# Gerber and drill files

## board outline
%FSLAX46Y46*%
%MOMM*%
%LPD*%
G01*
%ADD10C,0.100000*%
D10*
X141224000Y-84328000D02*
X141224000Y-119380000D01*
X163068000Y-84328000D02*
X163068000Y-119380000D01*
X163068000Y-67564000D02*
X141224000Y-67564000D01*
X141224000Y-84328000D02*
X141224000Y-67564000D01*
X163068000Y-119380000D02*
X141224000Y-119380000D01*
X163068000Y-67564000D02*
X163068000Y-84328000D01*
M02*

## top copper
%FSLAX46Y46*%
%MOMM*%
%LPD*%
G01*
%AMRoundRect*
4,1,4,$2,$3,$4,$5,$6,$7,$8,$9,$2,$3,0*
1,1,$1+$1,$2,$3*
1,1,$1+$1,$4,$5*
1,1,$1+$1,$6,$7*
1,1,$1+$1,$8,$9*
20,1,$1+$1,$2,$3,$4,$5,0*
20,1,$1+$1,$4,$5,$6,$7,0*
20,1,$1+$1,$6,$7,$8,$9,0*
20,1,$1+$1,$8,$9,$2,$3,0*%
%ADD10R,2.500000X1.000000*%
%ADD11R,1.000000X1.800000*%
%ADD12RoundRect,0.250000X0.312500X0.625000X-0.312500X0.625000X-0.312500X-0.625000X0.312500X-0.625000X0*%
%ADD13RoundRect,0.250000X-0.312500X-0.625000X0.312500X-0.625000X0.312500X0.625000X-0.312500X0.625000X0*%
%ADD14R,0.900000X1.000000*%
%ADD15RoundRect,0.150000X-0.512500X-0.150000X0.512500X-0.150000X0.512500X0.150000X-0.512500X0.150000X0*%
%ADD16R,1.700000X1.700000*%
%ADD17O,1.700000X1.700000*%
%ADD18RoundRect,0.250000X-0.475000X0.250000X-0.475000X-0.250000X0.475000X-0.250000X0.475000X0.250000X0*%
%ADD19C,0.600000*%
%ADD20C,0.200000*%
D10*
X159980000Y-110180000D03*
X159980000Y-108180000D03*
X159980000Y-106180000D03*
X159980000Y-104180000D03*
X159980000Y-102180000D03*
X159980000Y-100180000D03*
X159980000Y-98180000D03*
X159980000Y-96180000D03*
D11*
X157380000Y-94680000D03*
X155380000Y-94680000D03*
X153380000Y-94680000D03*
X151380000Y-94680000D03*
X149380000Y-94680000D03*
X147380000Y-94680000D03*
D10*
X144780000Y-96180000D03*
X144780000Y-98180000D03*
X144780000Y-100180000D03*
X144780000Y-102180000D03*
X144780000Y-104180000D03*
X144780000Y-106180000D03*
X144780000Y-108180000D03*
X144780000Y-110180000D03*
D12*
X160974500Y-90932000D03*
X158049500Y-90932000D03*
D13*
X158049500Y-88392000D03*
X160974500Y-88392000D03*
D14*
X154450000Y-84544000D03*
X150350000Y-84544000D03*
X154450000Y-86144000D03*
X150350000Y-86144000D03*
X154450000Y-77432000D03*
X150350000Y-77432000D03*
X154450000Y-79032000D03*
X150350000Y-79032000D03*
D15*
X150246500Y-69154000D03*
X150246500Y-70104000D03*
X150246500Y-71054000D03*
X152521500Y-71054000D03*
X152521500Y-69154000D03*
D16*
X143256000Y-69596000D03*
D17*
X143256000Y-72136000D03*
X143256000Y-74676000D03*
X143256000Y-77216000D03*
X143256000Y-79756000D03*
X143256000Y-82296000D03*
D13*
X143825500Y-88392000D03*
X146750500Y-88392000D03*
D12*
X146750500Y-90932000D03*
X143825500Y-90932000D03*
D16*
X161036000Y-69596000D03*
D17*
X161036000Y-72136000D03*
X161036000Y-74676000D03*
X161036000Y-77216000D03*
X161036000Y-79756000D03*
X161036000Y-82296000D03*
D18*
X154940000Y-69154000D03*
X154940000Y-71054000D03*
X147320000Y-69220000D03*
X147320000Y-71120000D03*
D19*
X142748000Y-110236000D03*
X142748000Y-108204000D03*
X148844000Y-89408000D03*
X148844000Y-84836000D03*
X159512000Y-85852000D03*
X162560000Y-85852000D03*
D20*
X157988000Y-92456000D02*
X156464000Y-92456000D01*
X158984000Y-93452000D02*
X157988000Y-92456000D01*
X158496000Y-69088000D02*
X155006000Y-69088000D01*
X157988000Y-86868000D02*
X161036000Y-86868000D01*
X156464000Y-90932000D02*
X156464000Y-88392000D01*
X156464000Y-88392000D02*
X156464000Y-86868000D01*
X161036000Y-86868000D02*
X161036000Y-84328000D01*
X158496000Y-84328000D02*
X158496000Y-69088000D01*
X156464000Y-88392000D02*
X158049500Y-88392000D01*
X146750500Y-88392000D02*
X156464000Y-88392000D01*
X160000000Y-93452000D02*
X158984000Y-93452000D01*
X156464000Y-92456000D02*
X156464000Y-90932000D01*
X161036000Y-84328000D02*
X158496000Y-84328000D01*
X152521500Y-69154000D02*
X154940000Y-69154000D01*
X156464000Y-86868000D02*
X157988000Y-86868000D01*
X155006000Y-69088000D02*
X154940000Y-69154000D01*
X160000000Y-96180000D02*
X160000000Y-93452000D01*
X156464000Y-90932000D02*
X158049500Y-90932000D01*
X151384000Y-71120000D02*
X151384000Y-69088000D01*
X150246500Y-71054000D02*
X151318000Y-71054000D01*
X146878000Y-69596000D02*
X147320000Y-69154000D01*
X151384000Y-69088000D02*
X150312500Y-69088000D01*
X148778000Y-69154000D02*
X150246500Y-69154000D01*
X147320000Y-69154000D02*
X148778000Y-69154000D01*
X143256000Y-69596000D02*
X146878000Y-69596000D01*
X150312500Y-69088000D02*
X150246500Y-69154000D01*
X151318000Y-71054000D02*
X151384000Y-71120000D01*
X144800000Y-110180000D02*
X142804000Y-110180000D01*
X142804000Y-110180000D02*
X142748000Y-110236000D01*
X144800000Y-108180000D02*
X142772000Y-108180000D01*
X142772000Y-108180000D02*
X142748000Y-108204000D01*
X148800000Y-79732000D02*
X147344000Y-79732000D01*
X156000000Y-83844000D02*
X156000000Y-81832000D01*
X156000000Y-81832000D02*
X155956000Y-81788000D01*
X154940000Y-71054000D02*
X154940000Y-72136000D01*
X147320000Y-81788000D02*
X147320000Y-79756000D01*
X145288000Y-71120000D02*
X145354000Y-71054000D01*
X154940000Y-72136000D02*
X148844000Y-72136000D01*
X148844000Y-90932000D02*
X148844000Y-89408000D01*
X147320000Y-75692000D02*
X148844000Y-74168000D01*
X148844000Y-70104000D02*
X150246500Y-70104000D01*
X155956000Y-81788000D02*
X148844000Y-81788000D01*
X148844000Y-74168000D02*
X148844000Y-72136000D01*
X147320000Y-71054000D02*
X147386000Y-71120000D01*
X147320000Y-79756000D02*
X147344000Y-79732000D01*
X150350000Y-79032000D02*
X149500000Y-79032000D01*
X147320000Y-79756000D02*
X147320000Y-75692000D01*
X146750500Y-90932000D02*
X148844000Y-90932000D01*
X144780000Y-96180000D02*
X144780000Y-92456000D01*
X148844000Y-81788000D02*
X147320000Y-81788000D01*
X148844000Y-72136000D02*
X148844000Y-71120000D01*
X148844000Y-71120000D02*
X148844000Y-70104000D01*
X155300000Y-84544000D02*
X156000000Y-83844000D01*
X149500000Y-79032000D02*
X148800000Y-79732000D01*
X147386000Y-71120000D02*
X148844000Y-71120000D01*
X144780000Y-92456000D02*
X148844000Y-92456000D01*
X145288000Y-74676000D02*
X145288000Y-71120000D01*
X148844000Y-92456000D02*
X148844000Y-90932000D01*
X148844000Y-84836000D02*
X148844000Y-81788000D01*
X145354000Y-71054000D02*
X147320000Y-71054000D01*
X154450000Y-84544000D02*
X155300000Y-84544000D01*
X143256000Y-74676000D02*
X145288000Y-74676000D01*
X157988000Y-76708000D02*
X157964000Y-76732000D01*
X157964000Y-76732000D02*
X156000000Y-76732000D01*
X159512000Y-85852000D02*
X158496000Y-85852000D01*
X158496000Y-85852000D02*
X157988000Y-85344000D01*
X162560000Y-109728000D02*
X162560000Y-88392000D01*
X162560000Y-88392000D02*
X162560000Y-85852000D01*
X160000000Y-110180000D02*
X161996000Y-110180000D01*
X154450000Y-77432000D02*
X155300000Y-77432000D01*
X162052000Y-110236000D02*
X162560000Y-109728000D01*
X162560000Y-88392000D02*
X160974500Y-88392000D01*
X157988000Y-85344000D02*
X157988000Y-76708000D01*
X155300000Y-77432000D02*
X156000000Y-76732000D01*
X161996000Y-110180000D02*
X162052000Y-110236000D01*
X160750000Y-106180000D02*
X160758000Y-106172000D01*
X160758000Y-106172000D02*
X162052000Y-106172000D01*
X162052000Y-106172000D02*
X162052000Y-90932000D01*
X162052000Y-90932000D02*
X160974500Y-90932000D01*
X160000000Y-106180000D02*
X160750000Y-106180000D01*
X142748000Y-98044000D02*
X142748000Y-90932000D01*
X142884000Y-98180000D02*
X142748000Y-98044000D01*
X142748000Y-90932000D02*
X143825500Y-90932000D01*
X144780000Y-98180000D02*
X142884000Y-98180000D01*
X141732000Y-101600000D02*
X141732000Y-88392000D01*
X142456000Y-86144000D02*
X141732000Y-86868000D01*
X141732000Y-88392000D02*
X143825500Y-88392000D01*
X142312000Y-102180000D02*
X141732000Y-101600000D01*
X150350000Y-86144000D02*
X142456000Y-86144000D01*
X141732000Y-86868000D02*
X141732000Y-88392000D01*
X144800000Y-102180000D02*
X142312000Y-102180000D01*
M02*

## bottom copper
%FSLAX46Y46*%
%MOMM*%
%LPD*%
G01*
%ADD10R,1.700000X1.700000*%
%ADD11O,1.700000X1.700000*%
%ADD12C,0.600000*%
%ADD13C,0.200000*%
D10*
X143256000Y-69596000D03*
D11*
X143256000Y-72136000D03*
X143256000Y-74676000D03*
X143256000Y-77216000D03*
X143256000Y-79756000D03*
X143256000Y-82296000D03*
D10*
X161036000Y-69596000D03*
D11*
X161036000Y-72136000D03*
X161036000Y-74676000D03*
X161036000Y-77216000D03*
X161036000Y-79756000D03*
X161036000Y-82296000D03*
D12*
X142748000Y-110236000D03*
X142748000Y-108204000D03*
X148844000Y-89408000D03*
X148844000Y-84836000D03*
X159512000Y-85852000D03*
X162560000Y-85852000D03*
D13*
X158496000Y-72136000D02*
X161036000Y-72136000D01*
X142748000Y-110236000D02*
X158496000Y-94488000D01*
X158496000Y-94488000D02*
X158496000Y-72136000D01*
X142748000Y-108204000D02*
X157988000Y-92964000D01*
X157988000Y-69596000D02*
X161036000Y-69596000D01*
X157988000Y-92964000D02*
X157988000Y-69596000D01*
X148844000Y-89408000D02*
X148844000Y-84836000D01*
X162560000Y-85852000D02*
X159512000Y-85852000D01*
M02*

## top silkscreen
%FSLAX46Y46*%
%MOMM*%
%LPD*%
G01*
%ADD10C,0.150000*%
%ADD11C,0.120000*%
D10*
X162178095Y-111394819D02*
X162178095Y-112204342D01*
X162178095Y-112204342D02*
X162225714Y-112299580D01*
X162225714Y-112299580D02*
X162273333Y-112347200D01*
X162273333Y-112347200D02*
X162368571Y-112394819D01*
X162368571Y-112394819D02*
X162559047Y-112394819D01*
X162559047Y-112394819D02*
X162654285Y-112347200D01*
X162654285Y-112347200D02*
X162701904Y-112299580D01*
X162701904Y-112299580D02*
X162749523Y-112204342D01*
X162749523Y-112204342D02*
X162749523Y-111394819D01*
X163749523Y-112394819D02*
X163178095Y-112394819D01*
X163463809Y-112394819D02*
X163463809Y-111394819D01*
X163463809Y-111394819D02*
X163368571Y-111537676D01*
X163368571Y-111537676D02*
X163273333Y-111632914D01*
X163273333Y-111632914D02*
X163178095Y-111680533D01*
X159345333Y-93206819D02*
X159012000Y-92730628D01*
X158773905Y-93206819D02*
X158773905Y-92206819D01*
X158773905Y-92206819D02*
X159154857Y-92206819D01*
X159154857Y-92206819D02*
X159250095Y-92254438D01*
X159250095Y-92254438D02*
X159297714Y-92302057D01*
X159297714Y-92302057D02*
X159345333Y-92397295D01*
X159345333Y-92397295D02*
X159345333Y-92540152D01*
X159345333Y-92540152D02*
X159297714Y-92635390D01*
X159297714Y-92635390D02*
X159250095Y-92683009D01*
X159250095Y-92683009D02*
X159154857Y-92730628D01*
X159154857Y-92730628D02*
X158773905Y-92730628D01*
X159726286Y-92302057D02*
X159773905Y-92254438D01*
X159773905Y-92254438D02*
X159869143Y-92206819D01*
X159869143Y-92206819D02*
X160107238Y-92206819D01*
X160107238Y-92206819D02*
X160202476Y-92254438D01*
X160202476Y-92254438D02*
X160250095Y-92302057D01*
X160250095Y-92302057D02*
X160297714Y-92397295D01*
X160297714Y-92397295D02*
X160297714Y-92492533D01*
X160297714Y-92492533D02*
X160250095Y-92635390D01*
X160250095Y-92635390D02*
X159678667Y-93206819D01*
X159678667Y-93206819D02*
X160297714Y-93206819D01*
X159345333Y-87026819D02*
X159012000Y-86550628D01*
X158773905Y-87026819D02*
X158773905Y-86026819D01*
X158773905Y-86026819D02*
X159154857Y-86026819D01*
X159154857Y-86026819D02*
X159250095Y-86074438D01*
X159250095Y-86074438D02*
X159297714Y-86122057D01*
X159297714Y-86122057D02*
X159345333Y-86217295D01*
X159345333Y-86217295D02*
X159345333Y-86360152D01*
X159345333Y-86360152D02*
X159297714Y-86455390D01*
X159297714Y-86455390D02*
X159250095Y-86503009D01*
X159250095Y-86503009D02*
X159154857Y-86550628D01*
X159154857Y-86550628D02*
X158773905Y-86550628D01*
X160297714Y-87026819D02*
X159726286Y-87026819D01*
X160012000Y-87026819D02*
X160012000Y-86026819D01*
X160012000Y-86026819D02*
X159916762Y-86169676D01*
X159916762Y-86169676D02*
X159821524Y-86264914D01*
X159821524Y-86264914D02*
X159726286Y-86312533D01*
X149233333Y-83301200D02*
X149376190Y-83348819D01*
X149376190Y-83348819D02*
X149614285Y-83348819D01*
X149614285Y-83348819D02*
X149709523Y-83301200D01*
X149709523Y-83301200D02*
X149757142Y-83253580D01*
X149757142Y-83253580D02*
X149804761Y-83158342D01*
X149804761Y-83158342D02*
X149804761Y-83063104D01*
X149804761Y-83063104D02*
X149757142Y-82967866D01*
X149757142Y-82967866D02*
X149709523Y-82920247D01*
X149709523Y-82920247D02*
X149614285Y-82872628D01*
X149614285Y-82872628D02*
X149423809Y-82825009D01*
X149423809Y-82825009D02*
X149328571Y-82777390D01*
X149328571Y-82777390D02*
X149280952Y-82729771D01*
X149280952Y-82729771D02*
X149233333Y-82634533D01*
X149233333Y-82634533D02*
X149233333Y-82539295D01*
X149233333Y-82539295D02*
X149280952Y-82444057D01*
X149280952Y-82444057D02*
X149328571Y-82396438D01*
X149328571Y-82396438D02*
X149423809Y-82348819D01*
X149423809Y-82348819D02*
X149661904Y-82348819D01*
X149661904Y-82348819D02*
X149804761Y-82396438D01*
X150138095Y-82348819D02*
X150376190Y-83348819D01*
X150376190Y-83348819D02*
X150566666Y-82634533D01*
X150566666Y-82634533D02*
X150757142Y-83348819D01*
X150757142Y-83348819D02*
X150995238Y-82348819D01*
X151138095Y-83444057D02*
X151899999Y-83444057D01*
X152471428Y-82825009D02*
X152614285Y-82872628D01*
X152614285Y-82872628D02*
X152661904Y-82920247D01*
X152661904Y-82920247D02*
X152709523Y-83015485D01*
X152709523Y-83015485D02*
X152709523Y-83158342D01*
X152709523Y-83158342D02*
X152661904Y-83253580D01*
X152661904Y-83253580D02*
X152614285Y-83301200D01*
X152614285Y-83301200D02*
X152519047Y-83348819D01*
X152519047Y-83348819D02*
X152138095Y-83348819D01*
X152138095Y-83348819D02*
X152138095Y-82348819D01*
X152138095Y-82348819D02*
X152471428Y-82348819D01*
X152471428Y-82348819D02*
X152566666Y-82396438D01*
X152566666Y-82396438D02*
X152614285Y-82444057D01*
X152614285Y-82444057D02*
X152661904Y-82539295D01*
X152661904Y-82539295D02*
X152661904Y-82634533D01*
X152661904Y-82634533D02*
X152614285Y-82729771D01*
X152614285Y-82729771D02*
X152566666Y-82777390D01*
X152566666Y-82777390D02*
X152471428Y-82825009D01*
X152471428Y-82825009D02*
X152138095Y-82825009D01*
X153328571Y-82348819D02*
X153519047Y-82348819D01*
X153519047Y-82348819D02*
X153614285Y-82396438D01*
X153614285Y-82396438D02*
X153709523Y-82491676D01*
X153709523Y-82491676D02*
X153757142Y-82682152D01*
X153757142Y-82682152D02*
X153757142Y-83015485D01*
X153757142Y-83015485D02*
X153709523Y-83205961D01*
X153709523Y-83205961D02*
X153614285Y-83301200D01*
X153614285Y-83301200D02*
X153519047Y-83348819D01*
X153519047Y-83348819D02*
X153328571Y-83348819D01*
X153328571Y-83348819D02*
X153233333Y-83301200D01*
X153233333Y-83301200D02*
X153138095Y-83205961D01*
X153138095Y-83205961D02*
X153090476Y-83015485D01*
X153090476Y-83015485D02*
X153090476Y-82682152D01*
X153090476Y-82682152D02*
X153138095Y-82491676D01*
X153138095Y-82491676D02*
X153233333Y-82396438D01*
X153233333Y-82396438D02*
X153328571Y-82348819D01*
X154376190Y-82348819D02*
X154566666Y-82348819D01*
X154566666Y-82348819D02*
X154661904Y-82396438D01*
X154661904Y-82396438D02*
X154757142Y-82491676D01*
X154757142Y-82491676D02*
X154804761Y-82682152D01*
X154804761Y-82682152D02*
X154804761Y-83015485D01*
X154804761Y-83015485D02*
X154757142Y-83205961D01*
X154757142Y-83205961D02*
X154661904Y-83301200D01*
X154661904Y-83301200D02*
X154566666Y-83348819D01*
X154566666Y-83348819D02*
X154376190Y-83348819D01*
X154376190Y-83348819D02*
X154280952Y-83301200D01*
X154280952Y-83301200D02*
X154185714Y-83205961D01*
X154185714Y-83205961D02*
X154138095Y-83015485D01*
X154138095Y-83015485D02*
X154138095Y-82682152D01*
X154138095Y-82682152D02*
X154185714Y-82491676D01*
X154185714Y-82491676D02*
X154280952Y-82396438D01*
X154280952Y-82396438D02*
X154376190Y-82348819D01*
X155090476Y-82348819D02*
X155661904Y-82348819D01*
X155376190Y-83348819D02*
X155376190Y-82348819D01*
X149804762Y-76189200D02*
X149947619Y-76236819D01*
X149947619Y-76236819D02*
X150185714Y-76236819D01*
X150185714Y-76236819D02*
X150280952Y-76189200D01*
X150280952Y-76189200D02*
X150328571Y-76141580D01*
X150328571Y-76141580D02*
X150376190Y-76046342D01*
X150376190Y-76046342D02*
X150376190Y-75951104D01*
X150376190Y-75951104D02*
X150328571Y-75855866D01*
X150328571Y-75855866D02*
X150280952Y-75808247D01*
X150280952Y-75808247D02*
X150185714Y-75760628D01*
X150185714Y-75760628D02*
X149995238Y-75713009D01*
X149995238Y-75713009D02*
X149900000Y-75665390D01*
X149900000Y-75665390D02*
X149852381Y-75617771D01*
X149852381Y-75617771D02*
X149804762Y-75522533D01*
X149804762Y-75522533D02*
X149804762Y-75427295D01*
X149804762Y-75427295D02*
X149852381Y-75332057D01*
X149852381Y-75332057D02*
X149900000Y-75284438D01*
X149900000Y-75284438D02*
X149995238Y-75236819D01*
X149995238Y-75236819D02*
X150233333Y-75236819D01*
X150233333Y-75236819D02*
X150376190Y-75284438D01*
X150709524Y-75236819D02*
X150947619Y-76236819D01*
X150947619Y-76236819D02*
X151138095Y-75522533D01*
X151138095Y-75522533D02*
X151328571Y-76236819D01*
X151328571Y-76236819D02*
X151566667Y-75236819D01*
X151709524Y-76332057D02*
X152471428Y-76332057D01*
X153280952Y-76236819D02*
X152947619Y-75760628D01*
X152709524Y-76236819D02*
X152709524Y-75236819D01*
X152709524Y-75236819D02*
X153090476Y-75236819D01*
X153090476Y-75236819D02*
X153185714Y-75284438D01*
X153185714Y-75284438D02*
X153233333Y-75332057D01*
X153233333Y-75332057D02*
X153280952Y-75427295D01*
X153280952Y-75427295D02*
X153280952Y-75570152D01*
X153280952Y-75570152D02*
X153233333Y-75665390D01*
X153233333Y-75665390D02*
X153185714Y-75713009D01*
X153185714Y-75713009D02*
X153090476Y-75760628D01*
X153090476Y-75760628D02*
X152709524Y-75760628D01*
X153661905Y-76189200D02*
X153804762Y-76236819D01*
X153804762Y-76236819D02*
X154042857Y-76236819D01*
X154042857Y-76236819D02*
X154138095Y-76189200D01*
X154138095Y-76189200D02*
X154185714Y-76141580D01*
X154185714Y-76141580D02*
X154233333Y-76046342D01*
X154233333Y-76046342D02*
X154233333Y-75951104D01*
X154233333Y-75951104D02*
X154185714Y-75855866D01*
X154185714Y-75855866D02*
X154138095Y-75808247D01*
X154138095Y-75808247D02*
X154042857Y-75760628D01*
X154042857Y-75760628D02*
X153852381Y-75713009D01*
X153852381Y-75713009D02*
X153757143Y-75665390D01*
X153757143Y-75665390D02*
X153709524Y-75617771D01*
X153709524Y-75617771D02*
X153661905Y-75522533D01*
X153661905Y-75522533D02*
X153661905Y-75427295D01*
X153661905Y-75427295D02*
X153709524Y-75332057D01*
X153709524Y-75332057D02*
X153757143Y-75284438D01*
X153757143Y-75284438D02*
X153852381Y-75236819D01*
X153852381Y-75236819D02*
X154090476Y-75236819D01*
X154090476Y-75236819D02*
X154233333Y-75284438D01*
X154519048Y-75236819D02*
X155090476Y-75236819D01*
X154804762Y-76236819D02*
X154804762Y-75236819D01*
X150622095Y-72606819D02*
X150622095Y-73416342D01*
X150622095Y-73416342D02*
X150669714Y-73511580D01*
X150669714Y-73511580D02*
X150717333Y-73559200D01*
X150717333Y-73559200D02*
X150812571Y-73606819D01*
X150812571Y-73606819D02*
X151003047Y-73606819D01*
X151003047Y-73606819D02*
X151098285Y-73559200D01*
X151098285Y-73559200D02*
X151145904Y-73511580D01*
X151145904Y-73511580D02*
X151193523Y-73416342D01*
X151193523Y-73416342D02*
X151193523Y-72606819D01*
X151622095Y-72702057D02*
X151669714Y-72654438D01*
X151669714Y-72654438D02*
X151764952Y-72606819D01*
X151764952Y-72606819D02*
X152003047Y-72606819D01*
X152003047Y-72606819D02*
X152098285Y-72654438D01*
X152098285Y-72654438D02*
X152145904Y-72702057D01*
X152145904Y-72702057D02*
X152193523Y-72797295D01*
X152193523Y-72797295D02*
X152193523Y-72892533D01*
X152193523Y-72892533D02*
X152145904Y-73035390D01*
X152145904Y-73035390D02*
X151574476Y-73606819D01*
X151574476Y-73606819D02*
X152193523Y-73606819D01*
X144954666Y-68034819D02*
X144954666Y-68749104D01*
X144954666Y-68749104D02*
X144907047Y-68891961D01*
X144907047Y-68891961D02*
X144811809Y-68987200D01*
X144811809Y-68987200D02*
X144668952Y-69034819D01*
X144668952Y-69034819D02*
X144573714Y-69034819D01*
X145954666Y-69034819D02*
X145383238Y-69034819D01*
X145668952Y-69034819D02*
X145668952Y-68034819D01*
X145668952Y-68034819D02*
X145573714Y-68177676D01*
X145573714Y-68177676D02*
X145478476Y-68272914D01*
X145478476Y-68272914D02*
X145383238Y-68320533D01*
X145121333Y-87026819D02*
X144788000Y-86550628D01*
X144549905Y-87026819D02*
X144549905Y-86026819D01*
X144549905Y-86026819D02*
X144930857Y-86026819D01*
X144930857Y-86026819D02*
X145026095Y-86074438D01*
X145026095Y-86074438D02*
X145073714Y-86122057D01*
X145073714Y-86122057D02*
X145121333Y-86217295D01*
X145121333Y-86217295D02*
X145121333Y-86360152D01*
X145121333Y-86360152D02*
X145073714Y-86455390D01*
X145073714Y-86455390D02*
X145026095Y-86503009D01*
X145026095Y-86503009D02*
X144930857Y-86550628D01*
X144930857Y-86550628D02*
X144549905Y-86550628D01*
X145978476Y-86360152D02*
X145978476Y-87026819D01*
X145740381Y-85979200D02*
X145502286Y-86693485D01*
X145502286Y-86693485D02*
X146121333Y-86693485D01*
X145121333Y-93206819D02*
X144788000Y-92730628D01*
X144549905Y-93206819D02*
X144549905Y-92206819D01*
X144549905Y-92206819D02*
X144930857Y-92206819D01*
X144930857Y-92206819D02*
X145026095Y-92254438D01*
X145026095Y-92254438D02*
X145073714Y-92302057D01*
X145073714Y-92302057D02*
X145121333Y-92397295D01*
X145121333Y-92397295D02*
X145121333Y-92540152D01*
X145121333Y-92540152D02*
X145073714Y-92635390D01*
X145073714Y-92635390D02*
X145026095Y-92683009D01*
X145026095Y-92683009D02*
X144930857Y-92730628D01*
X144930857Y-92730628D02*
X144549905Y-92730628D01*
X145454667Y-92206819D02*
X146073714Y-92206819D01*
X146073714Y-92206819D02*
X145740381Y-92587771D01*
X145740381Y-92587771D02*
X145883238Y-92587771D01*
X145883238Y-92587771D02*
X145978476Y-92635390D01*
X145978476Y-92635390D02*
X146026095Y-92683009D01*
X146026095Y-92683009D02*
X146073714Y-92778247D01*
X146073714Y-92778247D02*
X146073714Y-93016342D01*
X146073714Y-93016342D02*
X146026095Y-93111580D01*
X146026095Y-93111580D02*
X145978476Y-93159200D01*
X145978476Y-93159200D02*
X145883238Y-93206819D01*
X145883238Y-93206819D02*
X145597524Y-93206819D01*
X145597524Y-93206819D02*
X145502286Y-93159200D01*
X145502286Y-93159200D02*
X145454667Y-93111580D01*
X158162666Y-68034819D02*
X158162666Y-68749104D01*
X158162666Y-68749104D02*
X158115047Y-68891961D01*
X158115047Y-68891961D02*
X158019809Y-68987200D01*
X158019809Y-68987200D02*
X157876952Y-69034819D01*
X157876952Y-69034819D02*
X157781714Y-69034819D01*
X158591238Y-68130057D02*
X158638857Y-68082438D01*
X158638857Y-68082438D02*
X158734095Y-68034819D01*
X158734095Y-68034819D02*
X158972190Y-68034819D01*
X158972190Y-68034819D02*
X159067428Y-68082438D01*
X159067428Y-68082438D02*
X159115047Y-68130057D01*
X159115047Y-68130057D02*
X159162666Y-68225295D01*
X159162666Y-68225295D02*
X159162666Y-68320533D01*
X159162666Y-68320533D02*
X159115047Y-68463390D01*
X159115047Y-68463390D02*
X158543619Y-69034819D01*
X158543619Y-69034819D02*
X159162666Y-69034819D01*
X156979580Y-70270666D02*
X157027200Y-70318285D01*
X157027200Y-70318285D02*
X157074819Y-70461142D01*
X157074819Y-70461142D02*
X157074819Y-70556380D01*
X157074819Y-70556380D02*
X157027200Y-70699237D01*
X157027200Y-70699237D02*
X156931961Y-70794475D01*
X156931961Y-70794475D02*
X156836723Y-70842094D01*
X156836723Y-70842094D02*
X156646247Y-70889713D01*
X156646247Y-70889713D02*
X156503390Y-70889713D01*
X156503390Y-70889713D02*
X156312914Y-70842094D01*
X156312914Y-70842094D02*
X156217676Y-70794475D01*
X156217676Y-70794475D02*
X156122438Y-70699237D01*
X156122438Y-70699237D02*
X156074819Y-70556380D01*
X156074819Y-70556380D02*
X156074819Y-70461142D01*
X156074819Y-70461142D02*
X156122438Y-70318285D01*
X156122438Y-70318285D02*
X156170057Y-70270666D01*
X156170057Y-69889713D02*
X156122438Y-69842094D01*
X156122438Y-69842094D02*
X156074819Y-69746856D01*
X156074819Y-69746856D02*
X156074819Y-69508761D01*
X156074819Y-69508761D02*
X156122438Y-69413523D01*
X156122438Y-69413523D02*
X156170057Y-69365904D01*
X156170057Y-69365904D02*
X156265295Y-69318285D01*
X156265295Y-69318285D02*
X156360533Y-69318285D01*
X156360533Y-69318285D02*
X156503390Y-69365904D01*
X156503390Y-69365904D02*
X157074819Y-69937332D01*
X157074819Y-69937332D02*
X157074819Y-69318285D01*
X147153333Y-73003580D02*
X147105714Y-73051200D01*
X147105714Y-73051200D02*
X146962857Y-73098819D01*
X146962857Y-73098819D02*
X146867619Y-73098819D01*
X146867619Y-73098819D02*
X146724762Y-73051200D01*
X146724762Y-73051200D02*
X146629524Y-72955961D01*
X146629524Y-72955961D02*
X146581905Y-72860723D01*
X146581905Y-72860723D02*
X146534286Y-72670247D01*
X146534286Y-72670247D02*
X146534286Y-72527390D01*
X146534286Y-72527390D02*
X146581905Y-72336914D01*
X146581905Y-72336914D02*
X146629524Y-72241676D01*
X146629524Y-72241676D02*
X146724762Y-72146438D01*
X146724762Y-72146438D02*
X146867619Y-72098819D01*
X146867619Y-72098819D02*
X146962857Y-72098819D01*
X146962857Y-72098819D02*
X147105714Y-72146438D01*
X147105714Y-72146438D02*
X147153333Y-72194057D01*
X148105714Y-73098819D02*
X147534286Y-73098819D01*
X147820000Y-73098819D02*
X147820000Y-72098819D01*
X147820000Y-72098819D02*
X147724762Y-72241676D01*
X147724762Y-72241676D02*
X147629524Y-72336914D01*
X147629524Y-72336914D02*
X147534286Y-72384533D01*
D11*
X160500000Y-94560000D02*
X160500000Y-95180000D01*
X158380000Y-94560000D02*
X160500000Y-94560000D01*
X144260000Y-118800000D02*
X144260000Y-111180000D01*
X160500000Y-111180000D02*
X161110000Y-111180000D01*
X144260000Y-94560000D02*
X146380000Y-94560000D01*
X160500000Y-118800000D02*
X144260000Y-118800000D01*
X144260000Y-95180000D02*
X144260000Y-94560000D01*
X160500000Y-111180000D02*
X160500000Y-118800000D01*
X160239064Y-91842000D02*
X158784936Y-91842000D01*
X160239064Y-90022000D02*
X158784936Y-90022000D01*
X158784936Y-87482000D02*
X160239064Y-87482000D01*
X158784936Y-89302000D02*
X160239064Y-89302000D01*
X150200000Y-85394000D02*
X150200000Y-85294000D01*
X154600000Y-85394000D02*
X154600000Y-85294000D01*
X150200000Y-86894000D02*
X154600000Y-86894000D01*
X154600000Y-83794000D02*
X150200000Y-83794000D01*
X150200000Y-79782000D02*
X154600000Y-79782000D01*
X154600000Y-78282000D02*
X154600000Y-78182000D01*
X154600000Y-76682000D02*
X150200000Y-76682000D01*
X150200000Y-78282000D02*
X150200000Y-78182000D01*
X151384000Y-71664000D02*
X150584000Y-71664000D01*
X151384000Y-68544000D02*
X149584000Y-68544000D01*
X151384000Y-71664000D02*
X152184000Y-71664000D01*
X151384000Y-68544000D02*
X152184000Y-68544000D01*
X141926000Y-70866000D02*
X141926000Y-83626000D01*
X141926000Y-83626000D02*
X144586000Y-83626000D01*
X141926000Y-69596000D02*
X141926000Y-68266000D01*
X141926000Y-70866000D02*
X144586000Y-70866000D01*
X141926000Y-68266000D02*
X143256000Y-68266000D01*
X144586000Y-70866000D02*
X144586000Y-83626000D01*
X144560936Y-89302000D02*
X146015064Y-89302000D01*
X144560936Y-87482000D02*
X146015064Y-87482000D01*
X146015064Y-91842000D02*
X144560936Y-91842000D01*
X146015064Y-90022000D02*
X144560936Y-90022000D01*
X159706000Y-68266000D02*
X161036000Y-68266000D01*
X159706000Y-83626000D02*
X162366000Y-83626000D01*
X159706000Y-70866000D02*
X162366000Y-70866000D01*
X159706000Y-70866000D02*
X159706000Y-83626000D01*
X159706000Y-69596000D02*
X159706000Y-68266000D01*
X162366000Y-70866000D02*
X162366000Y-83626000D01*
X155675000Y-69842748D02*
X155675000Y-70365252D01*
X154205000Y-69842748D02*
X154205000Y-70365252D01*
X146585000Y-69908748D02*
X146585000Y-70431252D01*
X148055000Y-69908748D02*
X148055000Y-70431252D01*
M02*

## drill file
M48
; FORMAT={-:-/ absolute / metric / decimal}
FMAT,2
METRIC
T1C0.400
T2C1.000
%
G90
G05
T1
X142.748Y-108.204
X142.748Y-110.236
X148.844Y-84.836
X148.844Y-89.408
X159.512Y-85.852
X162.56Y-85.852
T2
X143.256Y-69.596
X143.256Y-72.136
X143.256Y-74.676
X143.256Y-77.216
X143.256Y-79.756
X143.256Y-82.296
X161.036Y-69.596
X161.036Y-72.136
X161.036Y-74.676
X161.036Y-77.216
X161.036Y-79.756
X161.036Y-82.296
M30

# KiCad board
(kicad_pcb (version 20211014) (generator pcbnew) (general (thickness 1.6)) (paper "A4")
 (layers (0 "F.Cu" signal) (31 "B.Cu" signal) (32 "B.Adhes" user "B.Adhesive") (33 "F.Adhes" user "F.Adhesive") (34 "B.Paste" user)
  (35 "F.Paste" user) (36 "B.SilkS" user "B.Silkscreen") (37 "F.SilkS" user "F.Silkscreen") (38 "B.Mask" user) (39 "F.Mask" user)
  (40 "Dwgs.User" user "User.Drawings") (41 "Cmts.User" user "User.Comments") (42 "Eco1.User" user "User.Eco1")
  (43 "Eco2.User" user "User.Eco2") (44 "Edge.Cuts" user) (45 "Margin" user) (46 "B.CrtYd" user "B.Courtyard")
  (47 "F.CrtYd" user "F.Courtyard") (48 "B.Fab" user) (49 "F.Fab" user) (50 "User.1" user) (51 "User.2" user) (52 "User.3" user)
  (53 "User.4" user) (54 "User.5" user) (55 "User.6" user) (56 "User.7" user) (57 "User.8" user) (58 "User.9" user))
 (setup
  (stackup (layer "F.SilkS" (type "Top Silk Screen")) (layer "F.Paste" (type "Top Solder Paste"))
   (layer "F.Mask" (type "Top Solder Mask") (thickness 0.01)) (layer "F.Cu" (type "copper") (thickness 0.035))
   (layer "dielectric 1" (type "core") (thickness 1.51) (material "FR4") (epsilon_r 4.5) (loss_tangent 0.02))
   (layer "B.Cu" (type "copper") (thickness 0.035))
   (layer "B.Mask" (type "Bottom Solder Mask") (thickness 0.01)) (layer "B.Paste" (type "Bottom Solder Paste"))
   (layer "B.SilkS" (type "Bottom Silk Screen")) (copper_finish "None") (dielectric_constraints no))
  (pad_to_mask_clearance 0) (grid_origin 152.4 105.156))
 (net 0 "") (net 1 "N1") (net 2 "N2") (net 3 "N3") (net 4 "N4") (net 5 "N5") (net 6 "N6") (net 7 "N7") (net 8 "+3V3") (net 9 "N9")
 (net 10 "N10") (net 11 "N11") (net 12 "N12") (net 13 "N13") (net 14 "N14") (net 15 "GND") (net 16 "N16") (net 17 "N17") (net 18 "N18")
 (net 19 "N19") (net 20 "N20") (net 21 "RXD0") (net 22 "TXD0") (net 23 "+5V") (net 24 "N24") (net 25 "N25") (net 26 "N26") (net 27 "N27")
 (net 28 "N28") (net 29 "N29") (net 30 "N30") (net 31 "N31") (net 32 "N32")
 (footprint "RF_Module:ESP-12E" (layer "F.Cu") (at 152.38 106.68 180)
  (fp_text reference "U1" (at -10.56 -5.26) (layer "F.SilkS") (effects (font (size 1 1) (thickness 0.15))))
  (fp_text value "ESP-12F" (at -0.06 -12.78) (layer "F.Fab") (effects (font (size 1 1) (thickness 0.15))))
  (fp_line (start -8.12 12.12) (end -8.12 11.5) (layer "F.SilkS") (width 0.12))
  (fp_line (start -6 12.12) (end -8.12 12.12) (layer "F.SilkS") (width 0.12))
  (fp_line (start 8.12 -12.12) (end 8.12 -4.5) (layer "F.SilkS") (width 0.12))
  (fp_line (start -8.12 -4.5) (end -8.73 -4.5) (layer "F.SilkS") (width 0.12))
  (fp_line (start 8.12 12.12) (end 6 12.12) (layer "F.SilkS") (width 0.12))
  (fp_line (start -8.12 -12.12) (end 8.12 -12.12) (layer "F.SilkS") (width 0.12))
  (fp_line (start 8.12 11.5) (end 8.12 12.12) (layer "F.SilkS") (width 0.12))
  (fp_line (start -8.12 -4.5) (end -8.12 -12.12) (layer "F.SilkS") (width 0.12))
  (pad "1" smd rect (at -7.6 -3.5 180) (size 2.5 1) (layers "F.Cu" "F.Paste" "F.Mask") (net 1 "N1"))
  (pad "2" smd rect (at -7.6 -1.5 180) (size 2.5 1) (layers "F.Cu" "F.Paste" "F.Mask") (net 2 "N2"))
  (pad "3" smd rect (at -7.6 0.5 180) (size 2.5 1) (layers "F.Cu" "F.Paste" "F.Mask") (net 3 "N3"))
  (pad "4" smd rect (at -7.6 2.5 180) (size 2.5 1) (layers "F.Cu" "F.Paste" "F.Mask") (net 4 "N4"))
  (pad "5" smd rect (at -7.6 4.5 180) (size 2.5 1) (layers "F.Cu" "F.Paste" "F.Mask") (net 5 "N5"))
  (pad "6" smd rect (at -7.6 6.5 180) (size 2.5 1) (layers "F.Cu" "F.Paste" "F.Mask") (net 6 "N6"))
  (pad "7" smd rect (at -7.6 8.5 180) (size 2.5 1) (layers "F.Cu" "F.Paste" "F.Mask") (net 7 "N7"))
  (pad "8" smd rect (at -7.6 10.5 180) (size 2.5 1) (layers "F.Cu" "F.Paste" "F.Mask") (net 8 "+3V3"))
  (pad "9" smd rect (at -5 12 180) (size 1 1.8) (layers "F.Cu" "F.Paste" "F.Mask") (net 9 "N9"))
  (pad "10" smd rect (at -3 12 180) (size 1 1.8) (layers "F.Cu" "F.Paste" "F.Mask") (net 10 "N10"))
  (pad "11" smd rect (at -1 12 180) (size 1 1.8) (layers "F.Cu" "F.Paste" "F.Mask") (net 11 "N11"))
  (pad "12" smd rect (at 1 12 180) (size 1 1.8) (layers "F.Cu" "F.Paste" "F.Mask") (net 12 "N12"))
  (pad "13" smd rect (at 3 12 180) (size 1 1.8) (layers "F.Cu" "F.Paste" "F.Mask") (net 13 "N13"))
  (pad "14" smd rect (at 5 12 180) (size 1 1.8) (layers "F.Cu" "F.Paste" "F.Mask") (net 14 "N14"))
  (pad "15" smd rect (at 7.6 10.5 180) (size 2.5 1) (layers "F.Cu" "F.Paste" "F.Mask") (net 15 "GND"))
  (pad "16" smd rect (at 7.6 8.5 180) (size 2.5 1) (layers "F.Cu" "F.Paste" "F.Mask") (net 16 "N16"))
  (pad "17" smd rect (at 7.6 6.5 180) (size 2.5 1) (layers "F.Cu" "F.Paste" "F.Mask") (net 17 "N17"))
  (pad "18" smd rect (at 7.6 4.5 180) (size 2.5 1) (layers "F.Cu" "F.Paste" "F.Mask") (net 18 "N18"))
  (pad "19" smd rect (at 7.6 2.5 180) (size 2.5 1) (layers "F.Cu" "F.Paste" "F.Mask") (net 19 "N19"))
  (pad "20" smd rect (at 7.6 0.5 180) (size 2.5 1) (layers "F.Cu" "F.Paste" "F.Mask") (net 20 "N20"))
  (pad "21" smd rect (at 7.6 -1.5 180) (size 2.5 1) (layers "F.Cu" "F.Paste" "F.Mask") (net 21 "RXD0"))
  (pad "22" smd rect (at 7.6 -3.5 180) (size 2.5 1) (layers "F.Cu" "F.Paste" "F.Mask") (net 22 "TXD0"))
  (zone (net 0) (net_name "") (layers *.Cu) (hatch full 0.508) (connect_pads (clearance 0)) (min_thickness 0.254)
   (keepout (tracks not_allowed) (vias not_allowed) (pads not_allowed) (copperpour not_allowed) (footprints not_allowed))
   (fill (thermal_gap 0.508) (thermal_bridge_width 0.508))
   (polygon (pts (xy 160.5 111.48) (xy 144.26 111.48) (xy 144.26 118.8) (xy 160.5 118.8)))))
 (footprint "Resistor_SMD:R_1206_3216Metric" (layer "F.Cu") (at 159.512 90.932 180)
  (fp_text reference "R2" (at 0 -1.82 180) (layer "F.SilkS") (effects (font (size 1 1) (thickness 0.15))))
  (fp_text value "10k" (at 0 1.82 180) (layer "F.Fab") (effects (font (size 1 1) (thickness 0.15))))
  (fp_line (start -0.727064 -0.91) (end 0.727064 -0.91) (layer "F.SilkS") (width 0.12))
  (fp_line (start -0.727064 0.91) (end 0.727064 0.91) (layer "F.SilkS") (width 0.12))
  (pad "1" smd roundrect (at -1.4625 0 180) (size 1.125 1.75) (layers "F.Cu" "F.Paste" "F.Mask") (roundrect_rratio 0.2222222222)
   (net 3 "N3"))
  (pad "2" smd roundrect (at 1.4625 0 180) (size 1.125 1.75) (layers "F.Cu" "F.Paste" "F.Mask") (roundrect_rratio 0.2222222222)
   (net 8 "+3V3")))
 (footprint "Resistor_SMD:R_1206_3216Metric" (layer "F.Cu") (at 159.512 88.392)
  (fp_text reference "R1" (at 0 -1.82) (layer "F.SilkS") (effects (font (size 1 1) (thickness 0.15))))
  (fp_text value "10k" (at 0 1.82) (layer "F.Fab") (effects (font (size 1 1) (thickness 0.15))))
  (fp_line (start -0.727064 -0.91) (end 0.727064 -0.91) (layer "F.SilkS") (width 0.12))
  (fp_line (start -0.727064 0.91) (end 0.727064 0.91) (layer "F.SilkS") (width 0.12))
  (pad "1" smd roundrect (at -1.4625 0) (size 1.125 1.75) (layers "F.Cu" "F.Paste" "F.Mask") (roundrect_rratio 0.2222222222) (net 8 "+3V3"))
  (pad "2" smd roundrect (at 1.4625 0) (size 1.125 1.75) (layers "F.Cu" "F.Paste" "F.Mask") (roundrect_rratio 0.2222222222) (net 1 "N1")))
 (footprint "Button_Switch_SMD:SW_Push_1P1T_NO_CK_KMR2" (layer "F.Cu") (at 152.4 85.344)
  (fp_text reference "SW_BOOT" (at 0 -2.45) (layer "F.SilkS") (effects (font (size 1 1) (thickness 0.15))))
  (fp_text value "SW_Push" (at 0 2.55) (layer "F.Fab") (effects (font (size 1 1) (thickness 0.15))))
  (fp_line (start -2.2 0.05) (end -2.2 -0.05) (layer "F.SilkS") (width 0.12))
  (fp_line (start 2.2 0.05) (end 2.2 -0.05) (layer "F.SilkS") (width 0.12))
  (fp_line (start -2.2 1.55) (end 2.2 1.55) (layer "F.SilkS") (width 0.12))
  (fp_line (start 2.2 -1.55) (end -2.2 -1.55) (layer "F.SilkS") (width 0.12))
  (pad "1" smd rect (at 2.05 -0.8) (size 0.9 1) (layers "F.Cu" "F.Paste" "F.Mask") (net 15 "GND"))
  (pad "1" smd rect (at -2.05 -0.8) (size 0.9 1) (layers "F.Cu" "F.Paste" "F.Mask") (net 15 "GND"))
  (pad "2" smd rect (at 2.05 0.8) (size 0.9 1) (layers "F.Cu" "F.Paste" "F.Mask") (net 18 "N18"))
  (pad "2" smd rect (at -2.05 0.8) (size 0.9 1) (layers "F.Cu" "F.Paste" "F.Mask") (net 18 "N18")))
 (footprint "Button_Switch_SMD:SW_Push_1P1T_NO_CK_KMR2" (layer "F.Cu") (at 152.4 78.232)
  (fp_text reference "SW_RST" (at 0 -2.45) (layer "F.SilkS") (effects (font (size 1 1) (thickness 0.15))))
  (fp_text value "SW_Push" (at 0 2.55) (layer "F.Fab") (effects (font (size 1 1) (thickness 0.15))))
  (fp_line (start -2.2 1.55) (end 2.2 1.55) (layer "F.SilkS") (width 0.12))
  (fp_line (start 2.2 0.05) (end 2.2 -0.05) (layer "F.SilkS") (width 0.12))
  (fp_line (start 2.2 -1.55) (end -2.2 -1.55) (layer "F.SilkS") (width 0.12))
  (fp_line (start -2.2 0.05) (end -2.2 -0.05) (layer "F.SilkS") (width 0.12))
  (pad "1" smd rect (at 2.05 -0.8) (size 0.9 1) (layers "F.Cu" "F.Paste" "F.Mask") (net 1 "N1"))
  (pad "1" smd rect (at -2.05 -0.8) (size 0.9 1) (layers "F.Cu" "F.Paste" "F.Mask") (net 1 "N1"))
  (pad "2" smd rect (at 2.05 0.8) (size 0.9 1) (layers "F.Cu" "F.Paste" "F.Mask") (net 15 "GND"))
  (pad "2" smd rect (at -2.05 0.8) (size 0.9 1) (layers "F.Cu" "F.Paste" "F.Mask") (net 15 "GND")))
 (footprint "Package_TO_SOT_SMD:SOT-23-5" (layer "F.Cu") (at 151.384 70.104)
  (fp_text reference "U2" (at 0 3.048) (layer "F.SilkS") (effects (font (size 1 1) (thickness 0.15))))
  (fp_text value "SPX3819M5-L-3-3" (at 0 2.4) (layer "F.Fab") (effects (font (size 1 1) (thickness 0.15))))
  (fp_line (start 0 1.56) (end -0.8 1.56) (layer "F.SilkS") (width 0.12))
  (fp_line (start 0 -1.56) (end -1.8 -1.56) (layer "F.SilkS") (width 0.12))
  (fp_line (start 0 1.56) (end 0.8 1.56) (layer "F.SilkS") (width 0.12))
  (fp_line (start 0 -1.56) (end 0.8 -1.56) (layer "F.SilkS") (width 0.12))
  (pad "1" smd roundrect (at -1.1375 -0.95) (size 1.325 0.6) (layers "F.Cu" "F.Paste" "F.Mask") (roundrect_rratio 0.25) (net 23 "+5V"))
  (pad "2" smd roundrect (at -1.1375 0) (size 1.325 0.6) (layers "F.Cu" "F.Paste" "F.Mask") (roundrect_rratio 0.25) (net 15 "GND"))
  (pad "3" smd roundrect (at -1.1375 0.95) (size 1.325 0.6) (layers "F.Cu" "F.Paste" "F.Mask") (roundrect_rratio 0.25) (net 23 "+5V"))
  (pad "4" smd roundrect (at 1.1375 0.95) (size 1.325 0.6) (layers "F.Cu" "F.Paste" "F.Mask") (roundrect_rratio 0.25) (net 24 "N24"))
  (pad "5" smd roundrect (at 1.1375 -0.95) (size 1.325 0.6) (layers "F.Cu" "F.Paste" "F.Mask") (roundrect_rratio 0.25) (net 8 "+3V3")))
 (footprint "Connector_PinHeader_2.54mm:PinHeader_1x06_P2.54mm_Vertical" (layer "F.Cu") (at 143.256 69.596)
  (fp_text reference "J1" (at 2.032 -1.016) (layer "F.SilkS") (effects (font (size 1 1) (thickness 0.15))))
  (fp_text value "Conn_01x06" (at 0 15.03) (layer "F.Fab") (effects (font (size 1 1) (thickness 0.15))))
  (fp_line (start -1.33 1.27) (end -1.33 14.03) (layer "F.SilkS") (width 0.12))
  (fp_line (start -1.33 14.03) (end 1.33 14.03) (layer "F.SilkS") (width 0.12))
  (fp_line (start -1.33 0) (end -1.33 -1.33) (layer "F.SilkS") (width 0.12))
  (fp_line (start -1.33 1.27) (end 1.33 1.27) (layer "F.SilkS") (width 0.12))
  (fp_line (start -1.33 -1.33) (end 0 -1.33) (layer "F.SilkS") (width 0.12))
  (fp_line (start 1.33 1.27) (end 1.33 14.03) (layer "F.SilkS") (width 0.12))
  (pad "1" thru_hole rect (at 0 0) (size 1.7 1.7) (drill 1) (layers *.Cu *.Mask) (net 23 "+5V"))
  (pad "2" thru_hole oval (at 0 2.54) (size 1.7 1.7) (drill 1) (layers *.Cu *.Mask) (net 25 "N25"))
  (pad "3" thru_hole oval (at 0 5.08) (size 1.7 1.7) (drill 1) (layers *.Cu *.Mask) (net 15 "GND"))
  (pad "4" thru_hole oval (at 0 7.62) (size 1.7 1.7) (drill 1) (layers *.Cu *.Mask) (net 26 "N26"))
  (pad "5" thru_hole oval (at 0 10.16) (size 1.7 1.7) (drill 1) (layers *.Cu *.Mask) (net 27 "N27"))
  (pad "6" thru_hole oval (at 0 12.7) (size 1.7 1.7) (drill 1) (layers *.Cu *.Mask) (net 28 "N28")))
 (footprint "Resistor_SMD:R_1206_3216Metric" (layer "F.Cu") (at 145.288 88.392)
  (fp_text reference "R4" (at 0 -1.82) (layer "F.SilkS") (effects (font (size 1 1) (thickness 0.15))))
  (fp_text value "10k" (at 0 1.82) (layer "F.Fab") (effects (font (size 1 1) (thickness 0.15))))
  (fp_line (start -0.727064 0.91) (end 0.727064 0.91) (layer "F.SilkS") (width 0.12))
  (fp_line (start -0.727064 -0.91) (end 0.727064 -0.91) (layer "F.SilkS") (width 0.12))
  (pad "1" smd roundrect (at -1.4625 0) (size 1.125 1.75) (layers "F.Cu" "F.Paste" "F.Mask") (roundrect_rratio 0.2222222222) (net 18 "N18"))
  (pad "2" smd roundrect (at 1.4625 0) (size 1.125 1.75) (layers "F.Cu" "F.Paste" "F.Mask") (roundrect_rratio 0.2222222222) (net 8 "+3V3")))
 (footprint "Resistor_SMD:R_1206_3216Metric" (layer "F.Cu") (at 145.288 90.932 180)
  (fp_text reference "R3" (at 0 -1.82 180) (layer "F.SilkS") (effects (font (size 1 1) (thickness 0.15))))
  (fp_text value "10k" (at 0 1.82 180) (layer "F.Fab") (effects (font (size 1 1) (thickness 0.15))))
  (fp_line (start -0.727064 -0.91) (end 0.727064 -0.91) (layer "F.SilkS") (width 0.12))
  (fp_line (start -0.727064 0.91) (end 0.727064 0.91) (layer "F.SilkS") (width 0.12))
  (pad "1" smd roundrect (at -1.4625 0 180) (size 1.125 1.75) (layers "F.Cu" "F.Paste" "F.Mask") (roundrect_rratio 0.2222222222)
   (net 15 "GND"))
  (pad "2" smd roundrect (at 1.4625 0 180) (size 1.125 1.75) (layers "F.Cu" "F.Paste" "F.Mask") (roundrect_rratio 0.2222222222)
   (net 16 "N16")))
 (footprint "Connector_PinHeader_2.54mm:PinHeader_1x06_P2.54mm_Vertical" (layer "F.Cu") (at 161.036 69.596)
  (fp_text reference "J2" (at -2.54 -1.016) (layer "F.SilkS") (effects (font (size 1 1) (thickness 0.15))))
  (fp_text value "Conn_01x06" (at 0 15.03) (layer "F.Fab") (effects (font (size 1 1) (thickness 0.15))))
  (fp_line (start -1.33 -1.33) (end 0 -1.33) (layer "F.SilkS") (width 0.12))
  (fp_line (start -1.33 14.03) (end 1.33 14.03) (layer "F.SilkS") (width 0.12))
  (fp_line (start -1.33 1.27) (end 1.33 1.27) (layer "F.SilkS") (width 0.12))
  (fp_line (start -1.33 1.27) (end -1.33 14.03) (layer "F.SilkS") (width 0.12))
  (fp_line (start -1.33 0) (end -1.33 -1.33) (layer "F.SilkS") (width 0.12))
  (fp_line (start 1.33 1.27) (end 1.33 14.03) (layer "F.SilkS") (width 0.12))
  (pad "1" thru_hole rect (at 0 0) (size 1.7 1.7) (drill 1) (layers *.Cu *.Mask) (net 21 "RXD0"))
  (pad "2" thru_hole oval (at 0 2.54) (size 1.7 1.7) (drill 1) (layers *.Cu *.Mask) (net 22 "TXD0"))
  (pad "3" thru_hole oval (at 0 5.08) (size 1.7 1.7) (drill 1) (layers *.Cu *.Mask) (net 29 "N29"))
  (pad "4" thru_hole oval (at 0 7.62) (size 1.7 1.7) (drill 1) (layers *.Cu *.Mask) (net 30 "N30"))
  (pad "5" thru_hole oval (at 0 10.16) (size 1.7 1.7) (drill 1) (layers *.Cu *.Mask) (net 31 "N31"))
  (pad "6" thru_hole oval (at 0 12.7) (size 1.7 1.7) (drill 1) (layers *.Cu *.Mask) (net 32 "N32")))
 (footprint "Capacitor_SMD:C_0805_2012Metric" (layer "F.Cu") (at 154.94 70.104 -90)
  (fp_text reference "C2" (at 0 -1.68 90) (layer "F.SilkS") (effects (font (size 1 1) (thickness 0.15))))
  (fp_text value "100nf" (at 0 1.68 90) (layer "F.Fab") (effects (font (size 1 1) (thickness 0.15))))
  (fp_line (start -0.261252 -0.735) (end 0.261252 -0.735) (layer "F.SilkS") (width 0.12))
  (fp_line (start -0.261252 0.735) (end 0.261252 0.735) (layer "F.SilkS") (width 0.12))
  (pad "1" smd roundrect (at -0.95 0 270) (size 1 1.45) (layers "F.Cu" "F.Paste" "F.Mask") (roundrect_rratio 0.25) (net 8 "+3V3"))
  (pad "2" smd roundrect (at 0.95 0 270) (size 1 1.45) (layers "F.Cu" "F.Paste" "F.Mask") (roundrect_rratio 0.25) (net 15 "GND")))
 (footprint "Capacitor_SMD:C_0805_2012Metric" (layer "F.Cu") (at 147.32 70.17 -90)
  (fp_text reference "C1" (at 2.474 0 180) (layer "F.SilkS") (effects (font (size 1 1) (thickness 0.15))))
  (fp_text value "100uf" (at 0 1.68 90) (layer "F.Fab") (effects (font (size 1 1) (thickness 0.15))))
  (fp_line (start -0.261252 0.735) (end 0.261252 0.735) (layer "F.SilkS") (width 0.12))
  (fp_line (start -0.261252 -0.735) (end 0.261252 -0.735) (layer "F.SilkS") (width 0.12))
  (pad "1" smd roundrect (at -0.95 0 270) (size 1 1.45) (layers "F.Cu" "F.Paste" "F.Mask") (roundrect_rratio 0.25) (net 23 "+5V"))
  (pad "2" smd roundrect (at 0.95 0 270) (size 1 1.45) (layers "F.Cu" "F.Paste" "F.Mask") (roundrect_rratio 0.25) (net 15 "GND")))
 (gr_line (start 141.224 84.328) (end 141.224 119.38) (layer "Edge.Cuts") (width 0.1))
 (gr_line (start 163.068 84.328) (end 163.068 119.38) (layer "Edge.Cuts") (width 0.1))
 (gr_line (start 163.068 67.564) (end 141.224 67.564) (layer "Edge.Cuts") (width 0.1))
 (gr_line (start 141.224 84.328) (end 141.224 67.564) (layer "Edge.Cuts") (width 0.1))
 (gr_line (start 163.068 119.38) (end 141.224 119.38) (layer "Edge.Cuts") (width 0.1))
 (gr_line (start 163.068 67.564) (end 163.068 84.328) (layer "Edge.Cuts") (width 0.1))
 (segment (start 157.988 92.456) (end 156.464 92.456) (width 0.2) (layer "F.Cu") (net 8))
 (segment (start 158.984 93.452) (end 157.988 92.456) (width 0.2) (layer "F.Cu") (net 8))
 (segment (start 158.496 69.088) (end 155.006 69.088) (width 0.2) (layer "F.Cu") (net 8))
 (segment (start 157.988 86.868) (end 161.036 86.868) (width 0.2) (layer "F.Cu") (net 8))
 (segment (start 156.464 90.932) (end 156.464 88.392) (width 0.2) (layer "F.Cu") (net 8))
 (segment (start 156.464 88.392) (end 156.464 86.868) (width 0.2) (layer "F.Cu") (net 8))
 (segment (start 161.036 86.868) (end 161.036 84.328) (width 0.2) (layer "F.Cu") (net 8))
 (segment (start 158.496 84.328) (end 158.496 69.088) (width 0.2) (layer "F.Cu") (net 8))
 (segment (start 156.464 88.392) (end 158.0495 88.392) (width 0.2) (layer "F.Cu") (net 8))
 (segment (start 146.7505 88.392) (end 156.464 88.392) (width 0.2) (layer "F.Cu") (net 8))
 (segment (start 160 93.452) (end 158.984 93.452) (width 0.2) (layer "F.Cu") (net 8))
 (segment (start 156.464 92.456) (end 156.464 90.932) (width 0.2) (layer "F.Cu") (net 8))
 (segment (start 161.036 84.328) (end 158.496 84.328) (width 0.2) (layer "F.Cu") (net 8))
 (segment (start 152.5215 69.154) (end 154.94 69.154) (width 0.2) (layer "F.Cu") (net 8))
 (segment (start 156.464 86.868) (end 157.988 86.868) (width 0.2) (layer "F.Cu") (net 8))
 (segment (start 155.006 69.088) (end 154.94 69.154) (width 0.2) (layer "F.Cu") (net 8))
 (segment (start 160 96.18) (end 160 93.452) (width 0.2) (layer "F.Cu") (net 8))
 (segment (start 156.464 90.932) (end 158.0495 90.932) (width 0.2) (layer "F.Cu") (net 8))
 (segment (start 151.384 71.12) (end 151.384 69.088) (width 0.2) (layer "F.Cu") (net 23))
 (segment (start 150.2465 71.054) (end 151.318 71.054) (width 0.2) (layer "F.Cu") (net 23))
 (segment (start 146.878 69.596) (end 147.32 69.154) (width 0.2) (layer "F.Cu") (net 23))
 (segment (start 151.384 69.088) (end 150.3125 69.088) (width 0.2) (layer "F.Cu") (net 23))
 (segment (start 148.778 69.154) (end 150.2465 69.154) (width 0.2) (layer "F.Cu") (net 23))
 (segment (start 147.32 69.154) (end 148.778 69.154) (width 0.2) (layer "F.Cu") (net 23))
 (segment (start 143.256 69.596) (end 146.878 69.596) (width 0.2) (layer "F.Cu") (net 23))
 (segment (start 150.3125 69.088) (end 150.2465 69.154) (width 0.2) (layer "F.Cu") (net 23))
 (segment (start 151.318 71.054) (end 151.384 71.12) (width 0.2) (layer "F.Cu") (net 23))
 (segment (start 144.8 110.18) (end 142.804 110.18) (width 0.2) (layer "F.Cu") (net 22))
 (segment (start 142.804 110.18) (end 142.748 110.236) (width 0.2) (layer "F.Cu") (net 22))
 (via (at 142.748 110.236) (size 0.6) (drill 0.4) (layers "F.Cu" "B.Cu") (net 22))
 (segment (start 158.496 72.136) (end 161.036 72.136) (width 0.2) (layer "B.Cu") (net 22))
 (segment (start 142.748 110.236) (end 158.496 94.488) (width 0.2) (layer "B.Cu") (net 22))
 (segment (start 158.496 94.488) (end 158.496 72.136) (width 0.2) (layer "B.Cu") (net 22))
 (segment (start 144.8 108.18) (end 142.772 108.18) (width 0.2) (layer "F.Cu") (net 21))
 (segment (start 142.772 108.18) (end 142.748 108.204) (width 0.2) (layer "F.Cu") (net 21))
 (via (at 142.748 108.204) (size 0.6) (drill 0.4) (layers "F.Cu" "B.Cu") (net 21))
 (segment (start 142.748 108.204) (end 157.988 92.964) (width 0.2) (layer "B.Cu") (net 21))
 (segment (start 157.988 69.596) (end 161.036 69.596) (width 0.2) (layer "B.Cu") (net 21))
 (segment (start 157.988 92.964) (end 157.988 69.596) (width 0.2) (layer "B.Cu") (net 21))
 (segment (start 148.8 79.732) (end 147.344 79.732) (width 0.2) (layer "F.Cu") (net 15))
 (segment (start 156 83.844) (end 156 81.832) (width 0.2) (layer "F.Cu") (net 15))
 (segment (start 156 81.832) (end 155.956 81.788) (width 0.2) (layer "F.Cu") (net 15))
 (segment (start 154.94 71.054) (end 154.94 72.136) (width 0.2) (layer "F.Cu") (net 15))
 (segment (start 147.32 81.788) (end 147.32 79.756) (width 0.2) (layer "F.Cu") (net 15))
 (segment (start 145.288 71.12) (end 145.354 71.054) (width 0.2) (layer "F.Cu") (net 15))
 (segment (start 154.94 72.136) (end 148.844 72.136) (width 0.2) (layer "F.Cu") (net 15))
 (segment (start 148.844 90.932) (end 148.844 89.408) (width 0.2) (layer "F.Cu") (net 15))
 (segment (start 147.32 75.692) (end 148.844 74.168) (width 0.2) (layer "F.Cu") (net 15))
 (segment (start 148.844 70.104) (end 150.2465 70.104) (width 0.2) (layer "F.Cu") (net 15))
 (segment (start 155.956 81.788) (end 148.844 81.788) (width 0.2) (layer "F.Cu") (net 15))
 (segment (start 148.844 74.168) (end 148.844 72.136) (width 0.2) (layer "F.Cu") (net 15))
 (segment (start 147.32 71.054) (end 147.386 71.12) (width 0.2) (layer "F.Cu") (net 15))
 (segment (start 147.32 79.756) (end 147.344 79.732) (width 0.2) (layer "F.Cu") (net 15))
 (segment (start 150.35 79.032) (end 149.5 79.032) (width 0.2) (layer "F.Cu") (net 15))
 (segment (start 147.32 79.756) (end 147.32 75.692) (width 0.2) (layer "F.Cu") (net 15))
 (segment (start 146.7505 90.932) (end 148.844 90.932) (width 0.2) (layer "F.Cu") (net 15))
 (segment (start 144.78 96.18) (end 144.78 92.456) (width 0.2) (layer "F.Cu") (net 15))
 (segment (start 148.844 81.788) (end 147.32 81.788) (width 0.2) (layer "F.Cu") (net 15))
 (segment (start 148.844 72.136) (end 148.844 71.12) (width 0.2) (layer "F.Cu") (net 15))
 (segment (start 148.844 71.12) (end 148.844 70.104) (width 0.2) (layer "F.Cu") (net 15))
 (segment (start 155.3 84.544) (end 156 83.844) (width 0.2) (layer "F.Cu") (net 15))
 (segment (start 149.5 79.032) (end 148.8 79.732) (width 0.2) (layer "F.Cu") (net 15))
 (segment (start 147.386 71.12) (end 148.844 71.12) (width 0.2) (layer "F.Cu") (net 15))
 (segment (start 144.78 92.456) (end 148.844 92.456) (width 0.2) (layer "F.Cu") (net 15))
 (segment (start 145.288 74.676) (end 145.288 71.12) (width 0.2) (layer "F.Cu") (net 15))
 (segment (start 148.844 92.456) (end 148.844 90.932) (width 0.2) (layer "F.Cu") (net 15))
 (segment (start 148.844 84.836) (end 148.844 81.788) (width 0.2) (layer "F.Cu") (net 15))
 (segment (start 145.354 71.054) (end 147.32 71.054) (width 0.2) (layer "F.Cu") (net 15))
 (segment (start 154.45 84.544) (end 155.3 84.544) (width 0.2) (layer "F.Cu") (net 15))
 (segment (start 143.256 74.676) (end 145.288 74.676) (width 0.2) (layer "F.Cu") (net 15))
 (via (at 148.844 89.408) (size 0.6) (drill 0.4) (layers "F.Cu" "B.Cu") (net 15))
 (via (at 148.844 84.836) (size 0.6) (drill 0.4) (layers "F.Cu" "B.Cu") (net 15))
 (segment (start 148.844 89.408) (end 148.844 84.836) (width 0.2) (layer "B.Cu") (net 15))
 (segment (start 157.988 76.708) (end 157.964 76.732) (width 0.2) (layer "F.Cu") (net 1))
 (segment (start 157.964 76.732) (end 156 76.732) (width 0.2) (layer "F.Cu") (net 1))
 (segment (start 159.512 85.852) (end 158.496 85.852) (width 0.2) (layer "F.Cu") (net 1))
 (segment (start 158.496 85.852) (end 157.988 85.344) (width 0.2) (layer "F.Cu") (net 1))
 (segment (start 162.56 109.728) (end 162.56 88.392) (width 0.2) (layer "F.Cu") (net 1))
 (segment (start 162.56 88.392) (end 162.56 85.852) (width 0.2) (layer "F.Cu") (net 1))
 (segment (start 160 110.18) (end 161.996 110.18) (width 0.2) (layer "F.Cu") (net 1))
 (segment (start 154.45 77.432) (end 155.3 77.432) (width 0.2) (layer "F.Cu") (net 1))
 (segment (start 162.052 110.236) (end 162.56 109.728) (width 0.2) (layer "F.Cu") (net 1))
 (segment (start 162.56 88.392) (end 160.9745 88.392) (width 0.2) (layer "F.Cu") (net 1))
 (segment (start 157.988 85.344) (end 157.988 76.708) (width 0.2) (layer "F.Cu") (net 1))
 (segment (start 155.3 77.432) (end 156 76.732) (width 0.2) (layer "F.Cu") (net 1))
 (segment (start 161.996 110.18) (end 162.052 110.236) (width 0.2) (layer "F.Cu") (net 1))
 (via (at 159.512 85.852) (size 0.6) (drill 0.4) (layers "F.Cu" "B.Cu") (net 1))
 (via (at 162.56 85.852) (size 0.6) (drill 0.4) (layers "F.Cu" "B.Cu") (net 1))
 (segment (start 162.56 85.852) (end 159.512 85.852) (width 0.2) (layer "B.Cu") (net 1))
 (segment (start 160.75 106.18) (end 160.758 106.172) (width 0.2) (layer "F.Cu") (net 3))
 (segment (start 160.758 106.172) (end 162.052 106.172) (width 0.2) (layer "F.Cu") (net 3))
 (segment (start 162.052 106.172) (end 162.052 90.932) (width 0.2) (layer "F.Cu") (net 3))
 (segment (start 162.052 90.932) (end 160.9745 90.932) (width 0.2) (layer "F.Cu") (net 3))
 (segment (start 160 106.18) (end 160.75 106.18) (width 0.2) (layer "F.Cu") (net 3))
 (segment (start 142.748 98.044) (end 142.748 90.932) (width 0.2) (layer "F.Cu") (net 16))
 (segment (start 142.884 98.18) (end 142.748 98.044) (width 0.2) (layer "F.Cu") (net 16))
 (segment (start 142.748 90.932) (end 143.8255 90.932) (width 0.2) (layer "F.Cu") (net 16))
 (segment (start 144.78 98.18) (end 142.884 98.18) (width 0.2) (layer "F.Cu") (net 16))
 (segment (start 141.732 101.6) (end 141.732 88.392) (width 0.2) (layer "F.Cu") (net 18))
 (segment (start 142.456 86.144) (end 141.732 86.868) (width 0.2) (layer "F.Cu") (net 18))
 (segment (start 141.732 88.392) (end 143.8255 88.392) (width 0.2) (layer "F.Cu") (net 18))
 (segment (start 142.312 102.18) (end 141.732 101.6) (width 0.2) (layer "F.Cu") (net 18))
 (segment (start 150.35 86.144) (end 142.456 86.144) (width 0.2) (layer "F.Cu") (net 18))
 (segment (start 141.732 86.868) (end 141.732 88.392) (width 0.2) (layer "F.Cu") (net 18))
 (segment (start 144.8 102.18) (end 142.312 102.18) (width 0.2) (layer "F.Cu") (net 18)))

